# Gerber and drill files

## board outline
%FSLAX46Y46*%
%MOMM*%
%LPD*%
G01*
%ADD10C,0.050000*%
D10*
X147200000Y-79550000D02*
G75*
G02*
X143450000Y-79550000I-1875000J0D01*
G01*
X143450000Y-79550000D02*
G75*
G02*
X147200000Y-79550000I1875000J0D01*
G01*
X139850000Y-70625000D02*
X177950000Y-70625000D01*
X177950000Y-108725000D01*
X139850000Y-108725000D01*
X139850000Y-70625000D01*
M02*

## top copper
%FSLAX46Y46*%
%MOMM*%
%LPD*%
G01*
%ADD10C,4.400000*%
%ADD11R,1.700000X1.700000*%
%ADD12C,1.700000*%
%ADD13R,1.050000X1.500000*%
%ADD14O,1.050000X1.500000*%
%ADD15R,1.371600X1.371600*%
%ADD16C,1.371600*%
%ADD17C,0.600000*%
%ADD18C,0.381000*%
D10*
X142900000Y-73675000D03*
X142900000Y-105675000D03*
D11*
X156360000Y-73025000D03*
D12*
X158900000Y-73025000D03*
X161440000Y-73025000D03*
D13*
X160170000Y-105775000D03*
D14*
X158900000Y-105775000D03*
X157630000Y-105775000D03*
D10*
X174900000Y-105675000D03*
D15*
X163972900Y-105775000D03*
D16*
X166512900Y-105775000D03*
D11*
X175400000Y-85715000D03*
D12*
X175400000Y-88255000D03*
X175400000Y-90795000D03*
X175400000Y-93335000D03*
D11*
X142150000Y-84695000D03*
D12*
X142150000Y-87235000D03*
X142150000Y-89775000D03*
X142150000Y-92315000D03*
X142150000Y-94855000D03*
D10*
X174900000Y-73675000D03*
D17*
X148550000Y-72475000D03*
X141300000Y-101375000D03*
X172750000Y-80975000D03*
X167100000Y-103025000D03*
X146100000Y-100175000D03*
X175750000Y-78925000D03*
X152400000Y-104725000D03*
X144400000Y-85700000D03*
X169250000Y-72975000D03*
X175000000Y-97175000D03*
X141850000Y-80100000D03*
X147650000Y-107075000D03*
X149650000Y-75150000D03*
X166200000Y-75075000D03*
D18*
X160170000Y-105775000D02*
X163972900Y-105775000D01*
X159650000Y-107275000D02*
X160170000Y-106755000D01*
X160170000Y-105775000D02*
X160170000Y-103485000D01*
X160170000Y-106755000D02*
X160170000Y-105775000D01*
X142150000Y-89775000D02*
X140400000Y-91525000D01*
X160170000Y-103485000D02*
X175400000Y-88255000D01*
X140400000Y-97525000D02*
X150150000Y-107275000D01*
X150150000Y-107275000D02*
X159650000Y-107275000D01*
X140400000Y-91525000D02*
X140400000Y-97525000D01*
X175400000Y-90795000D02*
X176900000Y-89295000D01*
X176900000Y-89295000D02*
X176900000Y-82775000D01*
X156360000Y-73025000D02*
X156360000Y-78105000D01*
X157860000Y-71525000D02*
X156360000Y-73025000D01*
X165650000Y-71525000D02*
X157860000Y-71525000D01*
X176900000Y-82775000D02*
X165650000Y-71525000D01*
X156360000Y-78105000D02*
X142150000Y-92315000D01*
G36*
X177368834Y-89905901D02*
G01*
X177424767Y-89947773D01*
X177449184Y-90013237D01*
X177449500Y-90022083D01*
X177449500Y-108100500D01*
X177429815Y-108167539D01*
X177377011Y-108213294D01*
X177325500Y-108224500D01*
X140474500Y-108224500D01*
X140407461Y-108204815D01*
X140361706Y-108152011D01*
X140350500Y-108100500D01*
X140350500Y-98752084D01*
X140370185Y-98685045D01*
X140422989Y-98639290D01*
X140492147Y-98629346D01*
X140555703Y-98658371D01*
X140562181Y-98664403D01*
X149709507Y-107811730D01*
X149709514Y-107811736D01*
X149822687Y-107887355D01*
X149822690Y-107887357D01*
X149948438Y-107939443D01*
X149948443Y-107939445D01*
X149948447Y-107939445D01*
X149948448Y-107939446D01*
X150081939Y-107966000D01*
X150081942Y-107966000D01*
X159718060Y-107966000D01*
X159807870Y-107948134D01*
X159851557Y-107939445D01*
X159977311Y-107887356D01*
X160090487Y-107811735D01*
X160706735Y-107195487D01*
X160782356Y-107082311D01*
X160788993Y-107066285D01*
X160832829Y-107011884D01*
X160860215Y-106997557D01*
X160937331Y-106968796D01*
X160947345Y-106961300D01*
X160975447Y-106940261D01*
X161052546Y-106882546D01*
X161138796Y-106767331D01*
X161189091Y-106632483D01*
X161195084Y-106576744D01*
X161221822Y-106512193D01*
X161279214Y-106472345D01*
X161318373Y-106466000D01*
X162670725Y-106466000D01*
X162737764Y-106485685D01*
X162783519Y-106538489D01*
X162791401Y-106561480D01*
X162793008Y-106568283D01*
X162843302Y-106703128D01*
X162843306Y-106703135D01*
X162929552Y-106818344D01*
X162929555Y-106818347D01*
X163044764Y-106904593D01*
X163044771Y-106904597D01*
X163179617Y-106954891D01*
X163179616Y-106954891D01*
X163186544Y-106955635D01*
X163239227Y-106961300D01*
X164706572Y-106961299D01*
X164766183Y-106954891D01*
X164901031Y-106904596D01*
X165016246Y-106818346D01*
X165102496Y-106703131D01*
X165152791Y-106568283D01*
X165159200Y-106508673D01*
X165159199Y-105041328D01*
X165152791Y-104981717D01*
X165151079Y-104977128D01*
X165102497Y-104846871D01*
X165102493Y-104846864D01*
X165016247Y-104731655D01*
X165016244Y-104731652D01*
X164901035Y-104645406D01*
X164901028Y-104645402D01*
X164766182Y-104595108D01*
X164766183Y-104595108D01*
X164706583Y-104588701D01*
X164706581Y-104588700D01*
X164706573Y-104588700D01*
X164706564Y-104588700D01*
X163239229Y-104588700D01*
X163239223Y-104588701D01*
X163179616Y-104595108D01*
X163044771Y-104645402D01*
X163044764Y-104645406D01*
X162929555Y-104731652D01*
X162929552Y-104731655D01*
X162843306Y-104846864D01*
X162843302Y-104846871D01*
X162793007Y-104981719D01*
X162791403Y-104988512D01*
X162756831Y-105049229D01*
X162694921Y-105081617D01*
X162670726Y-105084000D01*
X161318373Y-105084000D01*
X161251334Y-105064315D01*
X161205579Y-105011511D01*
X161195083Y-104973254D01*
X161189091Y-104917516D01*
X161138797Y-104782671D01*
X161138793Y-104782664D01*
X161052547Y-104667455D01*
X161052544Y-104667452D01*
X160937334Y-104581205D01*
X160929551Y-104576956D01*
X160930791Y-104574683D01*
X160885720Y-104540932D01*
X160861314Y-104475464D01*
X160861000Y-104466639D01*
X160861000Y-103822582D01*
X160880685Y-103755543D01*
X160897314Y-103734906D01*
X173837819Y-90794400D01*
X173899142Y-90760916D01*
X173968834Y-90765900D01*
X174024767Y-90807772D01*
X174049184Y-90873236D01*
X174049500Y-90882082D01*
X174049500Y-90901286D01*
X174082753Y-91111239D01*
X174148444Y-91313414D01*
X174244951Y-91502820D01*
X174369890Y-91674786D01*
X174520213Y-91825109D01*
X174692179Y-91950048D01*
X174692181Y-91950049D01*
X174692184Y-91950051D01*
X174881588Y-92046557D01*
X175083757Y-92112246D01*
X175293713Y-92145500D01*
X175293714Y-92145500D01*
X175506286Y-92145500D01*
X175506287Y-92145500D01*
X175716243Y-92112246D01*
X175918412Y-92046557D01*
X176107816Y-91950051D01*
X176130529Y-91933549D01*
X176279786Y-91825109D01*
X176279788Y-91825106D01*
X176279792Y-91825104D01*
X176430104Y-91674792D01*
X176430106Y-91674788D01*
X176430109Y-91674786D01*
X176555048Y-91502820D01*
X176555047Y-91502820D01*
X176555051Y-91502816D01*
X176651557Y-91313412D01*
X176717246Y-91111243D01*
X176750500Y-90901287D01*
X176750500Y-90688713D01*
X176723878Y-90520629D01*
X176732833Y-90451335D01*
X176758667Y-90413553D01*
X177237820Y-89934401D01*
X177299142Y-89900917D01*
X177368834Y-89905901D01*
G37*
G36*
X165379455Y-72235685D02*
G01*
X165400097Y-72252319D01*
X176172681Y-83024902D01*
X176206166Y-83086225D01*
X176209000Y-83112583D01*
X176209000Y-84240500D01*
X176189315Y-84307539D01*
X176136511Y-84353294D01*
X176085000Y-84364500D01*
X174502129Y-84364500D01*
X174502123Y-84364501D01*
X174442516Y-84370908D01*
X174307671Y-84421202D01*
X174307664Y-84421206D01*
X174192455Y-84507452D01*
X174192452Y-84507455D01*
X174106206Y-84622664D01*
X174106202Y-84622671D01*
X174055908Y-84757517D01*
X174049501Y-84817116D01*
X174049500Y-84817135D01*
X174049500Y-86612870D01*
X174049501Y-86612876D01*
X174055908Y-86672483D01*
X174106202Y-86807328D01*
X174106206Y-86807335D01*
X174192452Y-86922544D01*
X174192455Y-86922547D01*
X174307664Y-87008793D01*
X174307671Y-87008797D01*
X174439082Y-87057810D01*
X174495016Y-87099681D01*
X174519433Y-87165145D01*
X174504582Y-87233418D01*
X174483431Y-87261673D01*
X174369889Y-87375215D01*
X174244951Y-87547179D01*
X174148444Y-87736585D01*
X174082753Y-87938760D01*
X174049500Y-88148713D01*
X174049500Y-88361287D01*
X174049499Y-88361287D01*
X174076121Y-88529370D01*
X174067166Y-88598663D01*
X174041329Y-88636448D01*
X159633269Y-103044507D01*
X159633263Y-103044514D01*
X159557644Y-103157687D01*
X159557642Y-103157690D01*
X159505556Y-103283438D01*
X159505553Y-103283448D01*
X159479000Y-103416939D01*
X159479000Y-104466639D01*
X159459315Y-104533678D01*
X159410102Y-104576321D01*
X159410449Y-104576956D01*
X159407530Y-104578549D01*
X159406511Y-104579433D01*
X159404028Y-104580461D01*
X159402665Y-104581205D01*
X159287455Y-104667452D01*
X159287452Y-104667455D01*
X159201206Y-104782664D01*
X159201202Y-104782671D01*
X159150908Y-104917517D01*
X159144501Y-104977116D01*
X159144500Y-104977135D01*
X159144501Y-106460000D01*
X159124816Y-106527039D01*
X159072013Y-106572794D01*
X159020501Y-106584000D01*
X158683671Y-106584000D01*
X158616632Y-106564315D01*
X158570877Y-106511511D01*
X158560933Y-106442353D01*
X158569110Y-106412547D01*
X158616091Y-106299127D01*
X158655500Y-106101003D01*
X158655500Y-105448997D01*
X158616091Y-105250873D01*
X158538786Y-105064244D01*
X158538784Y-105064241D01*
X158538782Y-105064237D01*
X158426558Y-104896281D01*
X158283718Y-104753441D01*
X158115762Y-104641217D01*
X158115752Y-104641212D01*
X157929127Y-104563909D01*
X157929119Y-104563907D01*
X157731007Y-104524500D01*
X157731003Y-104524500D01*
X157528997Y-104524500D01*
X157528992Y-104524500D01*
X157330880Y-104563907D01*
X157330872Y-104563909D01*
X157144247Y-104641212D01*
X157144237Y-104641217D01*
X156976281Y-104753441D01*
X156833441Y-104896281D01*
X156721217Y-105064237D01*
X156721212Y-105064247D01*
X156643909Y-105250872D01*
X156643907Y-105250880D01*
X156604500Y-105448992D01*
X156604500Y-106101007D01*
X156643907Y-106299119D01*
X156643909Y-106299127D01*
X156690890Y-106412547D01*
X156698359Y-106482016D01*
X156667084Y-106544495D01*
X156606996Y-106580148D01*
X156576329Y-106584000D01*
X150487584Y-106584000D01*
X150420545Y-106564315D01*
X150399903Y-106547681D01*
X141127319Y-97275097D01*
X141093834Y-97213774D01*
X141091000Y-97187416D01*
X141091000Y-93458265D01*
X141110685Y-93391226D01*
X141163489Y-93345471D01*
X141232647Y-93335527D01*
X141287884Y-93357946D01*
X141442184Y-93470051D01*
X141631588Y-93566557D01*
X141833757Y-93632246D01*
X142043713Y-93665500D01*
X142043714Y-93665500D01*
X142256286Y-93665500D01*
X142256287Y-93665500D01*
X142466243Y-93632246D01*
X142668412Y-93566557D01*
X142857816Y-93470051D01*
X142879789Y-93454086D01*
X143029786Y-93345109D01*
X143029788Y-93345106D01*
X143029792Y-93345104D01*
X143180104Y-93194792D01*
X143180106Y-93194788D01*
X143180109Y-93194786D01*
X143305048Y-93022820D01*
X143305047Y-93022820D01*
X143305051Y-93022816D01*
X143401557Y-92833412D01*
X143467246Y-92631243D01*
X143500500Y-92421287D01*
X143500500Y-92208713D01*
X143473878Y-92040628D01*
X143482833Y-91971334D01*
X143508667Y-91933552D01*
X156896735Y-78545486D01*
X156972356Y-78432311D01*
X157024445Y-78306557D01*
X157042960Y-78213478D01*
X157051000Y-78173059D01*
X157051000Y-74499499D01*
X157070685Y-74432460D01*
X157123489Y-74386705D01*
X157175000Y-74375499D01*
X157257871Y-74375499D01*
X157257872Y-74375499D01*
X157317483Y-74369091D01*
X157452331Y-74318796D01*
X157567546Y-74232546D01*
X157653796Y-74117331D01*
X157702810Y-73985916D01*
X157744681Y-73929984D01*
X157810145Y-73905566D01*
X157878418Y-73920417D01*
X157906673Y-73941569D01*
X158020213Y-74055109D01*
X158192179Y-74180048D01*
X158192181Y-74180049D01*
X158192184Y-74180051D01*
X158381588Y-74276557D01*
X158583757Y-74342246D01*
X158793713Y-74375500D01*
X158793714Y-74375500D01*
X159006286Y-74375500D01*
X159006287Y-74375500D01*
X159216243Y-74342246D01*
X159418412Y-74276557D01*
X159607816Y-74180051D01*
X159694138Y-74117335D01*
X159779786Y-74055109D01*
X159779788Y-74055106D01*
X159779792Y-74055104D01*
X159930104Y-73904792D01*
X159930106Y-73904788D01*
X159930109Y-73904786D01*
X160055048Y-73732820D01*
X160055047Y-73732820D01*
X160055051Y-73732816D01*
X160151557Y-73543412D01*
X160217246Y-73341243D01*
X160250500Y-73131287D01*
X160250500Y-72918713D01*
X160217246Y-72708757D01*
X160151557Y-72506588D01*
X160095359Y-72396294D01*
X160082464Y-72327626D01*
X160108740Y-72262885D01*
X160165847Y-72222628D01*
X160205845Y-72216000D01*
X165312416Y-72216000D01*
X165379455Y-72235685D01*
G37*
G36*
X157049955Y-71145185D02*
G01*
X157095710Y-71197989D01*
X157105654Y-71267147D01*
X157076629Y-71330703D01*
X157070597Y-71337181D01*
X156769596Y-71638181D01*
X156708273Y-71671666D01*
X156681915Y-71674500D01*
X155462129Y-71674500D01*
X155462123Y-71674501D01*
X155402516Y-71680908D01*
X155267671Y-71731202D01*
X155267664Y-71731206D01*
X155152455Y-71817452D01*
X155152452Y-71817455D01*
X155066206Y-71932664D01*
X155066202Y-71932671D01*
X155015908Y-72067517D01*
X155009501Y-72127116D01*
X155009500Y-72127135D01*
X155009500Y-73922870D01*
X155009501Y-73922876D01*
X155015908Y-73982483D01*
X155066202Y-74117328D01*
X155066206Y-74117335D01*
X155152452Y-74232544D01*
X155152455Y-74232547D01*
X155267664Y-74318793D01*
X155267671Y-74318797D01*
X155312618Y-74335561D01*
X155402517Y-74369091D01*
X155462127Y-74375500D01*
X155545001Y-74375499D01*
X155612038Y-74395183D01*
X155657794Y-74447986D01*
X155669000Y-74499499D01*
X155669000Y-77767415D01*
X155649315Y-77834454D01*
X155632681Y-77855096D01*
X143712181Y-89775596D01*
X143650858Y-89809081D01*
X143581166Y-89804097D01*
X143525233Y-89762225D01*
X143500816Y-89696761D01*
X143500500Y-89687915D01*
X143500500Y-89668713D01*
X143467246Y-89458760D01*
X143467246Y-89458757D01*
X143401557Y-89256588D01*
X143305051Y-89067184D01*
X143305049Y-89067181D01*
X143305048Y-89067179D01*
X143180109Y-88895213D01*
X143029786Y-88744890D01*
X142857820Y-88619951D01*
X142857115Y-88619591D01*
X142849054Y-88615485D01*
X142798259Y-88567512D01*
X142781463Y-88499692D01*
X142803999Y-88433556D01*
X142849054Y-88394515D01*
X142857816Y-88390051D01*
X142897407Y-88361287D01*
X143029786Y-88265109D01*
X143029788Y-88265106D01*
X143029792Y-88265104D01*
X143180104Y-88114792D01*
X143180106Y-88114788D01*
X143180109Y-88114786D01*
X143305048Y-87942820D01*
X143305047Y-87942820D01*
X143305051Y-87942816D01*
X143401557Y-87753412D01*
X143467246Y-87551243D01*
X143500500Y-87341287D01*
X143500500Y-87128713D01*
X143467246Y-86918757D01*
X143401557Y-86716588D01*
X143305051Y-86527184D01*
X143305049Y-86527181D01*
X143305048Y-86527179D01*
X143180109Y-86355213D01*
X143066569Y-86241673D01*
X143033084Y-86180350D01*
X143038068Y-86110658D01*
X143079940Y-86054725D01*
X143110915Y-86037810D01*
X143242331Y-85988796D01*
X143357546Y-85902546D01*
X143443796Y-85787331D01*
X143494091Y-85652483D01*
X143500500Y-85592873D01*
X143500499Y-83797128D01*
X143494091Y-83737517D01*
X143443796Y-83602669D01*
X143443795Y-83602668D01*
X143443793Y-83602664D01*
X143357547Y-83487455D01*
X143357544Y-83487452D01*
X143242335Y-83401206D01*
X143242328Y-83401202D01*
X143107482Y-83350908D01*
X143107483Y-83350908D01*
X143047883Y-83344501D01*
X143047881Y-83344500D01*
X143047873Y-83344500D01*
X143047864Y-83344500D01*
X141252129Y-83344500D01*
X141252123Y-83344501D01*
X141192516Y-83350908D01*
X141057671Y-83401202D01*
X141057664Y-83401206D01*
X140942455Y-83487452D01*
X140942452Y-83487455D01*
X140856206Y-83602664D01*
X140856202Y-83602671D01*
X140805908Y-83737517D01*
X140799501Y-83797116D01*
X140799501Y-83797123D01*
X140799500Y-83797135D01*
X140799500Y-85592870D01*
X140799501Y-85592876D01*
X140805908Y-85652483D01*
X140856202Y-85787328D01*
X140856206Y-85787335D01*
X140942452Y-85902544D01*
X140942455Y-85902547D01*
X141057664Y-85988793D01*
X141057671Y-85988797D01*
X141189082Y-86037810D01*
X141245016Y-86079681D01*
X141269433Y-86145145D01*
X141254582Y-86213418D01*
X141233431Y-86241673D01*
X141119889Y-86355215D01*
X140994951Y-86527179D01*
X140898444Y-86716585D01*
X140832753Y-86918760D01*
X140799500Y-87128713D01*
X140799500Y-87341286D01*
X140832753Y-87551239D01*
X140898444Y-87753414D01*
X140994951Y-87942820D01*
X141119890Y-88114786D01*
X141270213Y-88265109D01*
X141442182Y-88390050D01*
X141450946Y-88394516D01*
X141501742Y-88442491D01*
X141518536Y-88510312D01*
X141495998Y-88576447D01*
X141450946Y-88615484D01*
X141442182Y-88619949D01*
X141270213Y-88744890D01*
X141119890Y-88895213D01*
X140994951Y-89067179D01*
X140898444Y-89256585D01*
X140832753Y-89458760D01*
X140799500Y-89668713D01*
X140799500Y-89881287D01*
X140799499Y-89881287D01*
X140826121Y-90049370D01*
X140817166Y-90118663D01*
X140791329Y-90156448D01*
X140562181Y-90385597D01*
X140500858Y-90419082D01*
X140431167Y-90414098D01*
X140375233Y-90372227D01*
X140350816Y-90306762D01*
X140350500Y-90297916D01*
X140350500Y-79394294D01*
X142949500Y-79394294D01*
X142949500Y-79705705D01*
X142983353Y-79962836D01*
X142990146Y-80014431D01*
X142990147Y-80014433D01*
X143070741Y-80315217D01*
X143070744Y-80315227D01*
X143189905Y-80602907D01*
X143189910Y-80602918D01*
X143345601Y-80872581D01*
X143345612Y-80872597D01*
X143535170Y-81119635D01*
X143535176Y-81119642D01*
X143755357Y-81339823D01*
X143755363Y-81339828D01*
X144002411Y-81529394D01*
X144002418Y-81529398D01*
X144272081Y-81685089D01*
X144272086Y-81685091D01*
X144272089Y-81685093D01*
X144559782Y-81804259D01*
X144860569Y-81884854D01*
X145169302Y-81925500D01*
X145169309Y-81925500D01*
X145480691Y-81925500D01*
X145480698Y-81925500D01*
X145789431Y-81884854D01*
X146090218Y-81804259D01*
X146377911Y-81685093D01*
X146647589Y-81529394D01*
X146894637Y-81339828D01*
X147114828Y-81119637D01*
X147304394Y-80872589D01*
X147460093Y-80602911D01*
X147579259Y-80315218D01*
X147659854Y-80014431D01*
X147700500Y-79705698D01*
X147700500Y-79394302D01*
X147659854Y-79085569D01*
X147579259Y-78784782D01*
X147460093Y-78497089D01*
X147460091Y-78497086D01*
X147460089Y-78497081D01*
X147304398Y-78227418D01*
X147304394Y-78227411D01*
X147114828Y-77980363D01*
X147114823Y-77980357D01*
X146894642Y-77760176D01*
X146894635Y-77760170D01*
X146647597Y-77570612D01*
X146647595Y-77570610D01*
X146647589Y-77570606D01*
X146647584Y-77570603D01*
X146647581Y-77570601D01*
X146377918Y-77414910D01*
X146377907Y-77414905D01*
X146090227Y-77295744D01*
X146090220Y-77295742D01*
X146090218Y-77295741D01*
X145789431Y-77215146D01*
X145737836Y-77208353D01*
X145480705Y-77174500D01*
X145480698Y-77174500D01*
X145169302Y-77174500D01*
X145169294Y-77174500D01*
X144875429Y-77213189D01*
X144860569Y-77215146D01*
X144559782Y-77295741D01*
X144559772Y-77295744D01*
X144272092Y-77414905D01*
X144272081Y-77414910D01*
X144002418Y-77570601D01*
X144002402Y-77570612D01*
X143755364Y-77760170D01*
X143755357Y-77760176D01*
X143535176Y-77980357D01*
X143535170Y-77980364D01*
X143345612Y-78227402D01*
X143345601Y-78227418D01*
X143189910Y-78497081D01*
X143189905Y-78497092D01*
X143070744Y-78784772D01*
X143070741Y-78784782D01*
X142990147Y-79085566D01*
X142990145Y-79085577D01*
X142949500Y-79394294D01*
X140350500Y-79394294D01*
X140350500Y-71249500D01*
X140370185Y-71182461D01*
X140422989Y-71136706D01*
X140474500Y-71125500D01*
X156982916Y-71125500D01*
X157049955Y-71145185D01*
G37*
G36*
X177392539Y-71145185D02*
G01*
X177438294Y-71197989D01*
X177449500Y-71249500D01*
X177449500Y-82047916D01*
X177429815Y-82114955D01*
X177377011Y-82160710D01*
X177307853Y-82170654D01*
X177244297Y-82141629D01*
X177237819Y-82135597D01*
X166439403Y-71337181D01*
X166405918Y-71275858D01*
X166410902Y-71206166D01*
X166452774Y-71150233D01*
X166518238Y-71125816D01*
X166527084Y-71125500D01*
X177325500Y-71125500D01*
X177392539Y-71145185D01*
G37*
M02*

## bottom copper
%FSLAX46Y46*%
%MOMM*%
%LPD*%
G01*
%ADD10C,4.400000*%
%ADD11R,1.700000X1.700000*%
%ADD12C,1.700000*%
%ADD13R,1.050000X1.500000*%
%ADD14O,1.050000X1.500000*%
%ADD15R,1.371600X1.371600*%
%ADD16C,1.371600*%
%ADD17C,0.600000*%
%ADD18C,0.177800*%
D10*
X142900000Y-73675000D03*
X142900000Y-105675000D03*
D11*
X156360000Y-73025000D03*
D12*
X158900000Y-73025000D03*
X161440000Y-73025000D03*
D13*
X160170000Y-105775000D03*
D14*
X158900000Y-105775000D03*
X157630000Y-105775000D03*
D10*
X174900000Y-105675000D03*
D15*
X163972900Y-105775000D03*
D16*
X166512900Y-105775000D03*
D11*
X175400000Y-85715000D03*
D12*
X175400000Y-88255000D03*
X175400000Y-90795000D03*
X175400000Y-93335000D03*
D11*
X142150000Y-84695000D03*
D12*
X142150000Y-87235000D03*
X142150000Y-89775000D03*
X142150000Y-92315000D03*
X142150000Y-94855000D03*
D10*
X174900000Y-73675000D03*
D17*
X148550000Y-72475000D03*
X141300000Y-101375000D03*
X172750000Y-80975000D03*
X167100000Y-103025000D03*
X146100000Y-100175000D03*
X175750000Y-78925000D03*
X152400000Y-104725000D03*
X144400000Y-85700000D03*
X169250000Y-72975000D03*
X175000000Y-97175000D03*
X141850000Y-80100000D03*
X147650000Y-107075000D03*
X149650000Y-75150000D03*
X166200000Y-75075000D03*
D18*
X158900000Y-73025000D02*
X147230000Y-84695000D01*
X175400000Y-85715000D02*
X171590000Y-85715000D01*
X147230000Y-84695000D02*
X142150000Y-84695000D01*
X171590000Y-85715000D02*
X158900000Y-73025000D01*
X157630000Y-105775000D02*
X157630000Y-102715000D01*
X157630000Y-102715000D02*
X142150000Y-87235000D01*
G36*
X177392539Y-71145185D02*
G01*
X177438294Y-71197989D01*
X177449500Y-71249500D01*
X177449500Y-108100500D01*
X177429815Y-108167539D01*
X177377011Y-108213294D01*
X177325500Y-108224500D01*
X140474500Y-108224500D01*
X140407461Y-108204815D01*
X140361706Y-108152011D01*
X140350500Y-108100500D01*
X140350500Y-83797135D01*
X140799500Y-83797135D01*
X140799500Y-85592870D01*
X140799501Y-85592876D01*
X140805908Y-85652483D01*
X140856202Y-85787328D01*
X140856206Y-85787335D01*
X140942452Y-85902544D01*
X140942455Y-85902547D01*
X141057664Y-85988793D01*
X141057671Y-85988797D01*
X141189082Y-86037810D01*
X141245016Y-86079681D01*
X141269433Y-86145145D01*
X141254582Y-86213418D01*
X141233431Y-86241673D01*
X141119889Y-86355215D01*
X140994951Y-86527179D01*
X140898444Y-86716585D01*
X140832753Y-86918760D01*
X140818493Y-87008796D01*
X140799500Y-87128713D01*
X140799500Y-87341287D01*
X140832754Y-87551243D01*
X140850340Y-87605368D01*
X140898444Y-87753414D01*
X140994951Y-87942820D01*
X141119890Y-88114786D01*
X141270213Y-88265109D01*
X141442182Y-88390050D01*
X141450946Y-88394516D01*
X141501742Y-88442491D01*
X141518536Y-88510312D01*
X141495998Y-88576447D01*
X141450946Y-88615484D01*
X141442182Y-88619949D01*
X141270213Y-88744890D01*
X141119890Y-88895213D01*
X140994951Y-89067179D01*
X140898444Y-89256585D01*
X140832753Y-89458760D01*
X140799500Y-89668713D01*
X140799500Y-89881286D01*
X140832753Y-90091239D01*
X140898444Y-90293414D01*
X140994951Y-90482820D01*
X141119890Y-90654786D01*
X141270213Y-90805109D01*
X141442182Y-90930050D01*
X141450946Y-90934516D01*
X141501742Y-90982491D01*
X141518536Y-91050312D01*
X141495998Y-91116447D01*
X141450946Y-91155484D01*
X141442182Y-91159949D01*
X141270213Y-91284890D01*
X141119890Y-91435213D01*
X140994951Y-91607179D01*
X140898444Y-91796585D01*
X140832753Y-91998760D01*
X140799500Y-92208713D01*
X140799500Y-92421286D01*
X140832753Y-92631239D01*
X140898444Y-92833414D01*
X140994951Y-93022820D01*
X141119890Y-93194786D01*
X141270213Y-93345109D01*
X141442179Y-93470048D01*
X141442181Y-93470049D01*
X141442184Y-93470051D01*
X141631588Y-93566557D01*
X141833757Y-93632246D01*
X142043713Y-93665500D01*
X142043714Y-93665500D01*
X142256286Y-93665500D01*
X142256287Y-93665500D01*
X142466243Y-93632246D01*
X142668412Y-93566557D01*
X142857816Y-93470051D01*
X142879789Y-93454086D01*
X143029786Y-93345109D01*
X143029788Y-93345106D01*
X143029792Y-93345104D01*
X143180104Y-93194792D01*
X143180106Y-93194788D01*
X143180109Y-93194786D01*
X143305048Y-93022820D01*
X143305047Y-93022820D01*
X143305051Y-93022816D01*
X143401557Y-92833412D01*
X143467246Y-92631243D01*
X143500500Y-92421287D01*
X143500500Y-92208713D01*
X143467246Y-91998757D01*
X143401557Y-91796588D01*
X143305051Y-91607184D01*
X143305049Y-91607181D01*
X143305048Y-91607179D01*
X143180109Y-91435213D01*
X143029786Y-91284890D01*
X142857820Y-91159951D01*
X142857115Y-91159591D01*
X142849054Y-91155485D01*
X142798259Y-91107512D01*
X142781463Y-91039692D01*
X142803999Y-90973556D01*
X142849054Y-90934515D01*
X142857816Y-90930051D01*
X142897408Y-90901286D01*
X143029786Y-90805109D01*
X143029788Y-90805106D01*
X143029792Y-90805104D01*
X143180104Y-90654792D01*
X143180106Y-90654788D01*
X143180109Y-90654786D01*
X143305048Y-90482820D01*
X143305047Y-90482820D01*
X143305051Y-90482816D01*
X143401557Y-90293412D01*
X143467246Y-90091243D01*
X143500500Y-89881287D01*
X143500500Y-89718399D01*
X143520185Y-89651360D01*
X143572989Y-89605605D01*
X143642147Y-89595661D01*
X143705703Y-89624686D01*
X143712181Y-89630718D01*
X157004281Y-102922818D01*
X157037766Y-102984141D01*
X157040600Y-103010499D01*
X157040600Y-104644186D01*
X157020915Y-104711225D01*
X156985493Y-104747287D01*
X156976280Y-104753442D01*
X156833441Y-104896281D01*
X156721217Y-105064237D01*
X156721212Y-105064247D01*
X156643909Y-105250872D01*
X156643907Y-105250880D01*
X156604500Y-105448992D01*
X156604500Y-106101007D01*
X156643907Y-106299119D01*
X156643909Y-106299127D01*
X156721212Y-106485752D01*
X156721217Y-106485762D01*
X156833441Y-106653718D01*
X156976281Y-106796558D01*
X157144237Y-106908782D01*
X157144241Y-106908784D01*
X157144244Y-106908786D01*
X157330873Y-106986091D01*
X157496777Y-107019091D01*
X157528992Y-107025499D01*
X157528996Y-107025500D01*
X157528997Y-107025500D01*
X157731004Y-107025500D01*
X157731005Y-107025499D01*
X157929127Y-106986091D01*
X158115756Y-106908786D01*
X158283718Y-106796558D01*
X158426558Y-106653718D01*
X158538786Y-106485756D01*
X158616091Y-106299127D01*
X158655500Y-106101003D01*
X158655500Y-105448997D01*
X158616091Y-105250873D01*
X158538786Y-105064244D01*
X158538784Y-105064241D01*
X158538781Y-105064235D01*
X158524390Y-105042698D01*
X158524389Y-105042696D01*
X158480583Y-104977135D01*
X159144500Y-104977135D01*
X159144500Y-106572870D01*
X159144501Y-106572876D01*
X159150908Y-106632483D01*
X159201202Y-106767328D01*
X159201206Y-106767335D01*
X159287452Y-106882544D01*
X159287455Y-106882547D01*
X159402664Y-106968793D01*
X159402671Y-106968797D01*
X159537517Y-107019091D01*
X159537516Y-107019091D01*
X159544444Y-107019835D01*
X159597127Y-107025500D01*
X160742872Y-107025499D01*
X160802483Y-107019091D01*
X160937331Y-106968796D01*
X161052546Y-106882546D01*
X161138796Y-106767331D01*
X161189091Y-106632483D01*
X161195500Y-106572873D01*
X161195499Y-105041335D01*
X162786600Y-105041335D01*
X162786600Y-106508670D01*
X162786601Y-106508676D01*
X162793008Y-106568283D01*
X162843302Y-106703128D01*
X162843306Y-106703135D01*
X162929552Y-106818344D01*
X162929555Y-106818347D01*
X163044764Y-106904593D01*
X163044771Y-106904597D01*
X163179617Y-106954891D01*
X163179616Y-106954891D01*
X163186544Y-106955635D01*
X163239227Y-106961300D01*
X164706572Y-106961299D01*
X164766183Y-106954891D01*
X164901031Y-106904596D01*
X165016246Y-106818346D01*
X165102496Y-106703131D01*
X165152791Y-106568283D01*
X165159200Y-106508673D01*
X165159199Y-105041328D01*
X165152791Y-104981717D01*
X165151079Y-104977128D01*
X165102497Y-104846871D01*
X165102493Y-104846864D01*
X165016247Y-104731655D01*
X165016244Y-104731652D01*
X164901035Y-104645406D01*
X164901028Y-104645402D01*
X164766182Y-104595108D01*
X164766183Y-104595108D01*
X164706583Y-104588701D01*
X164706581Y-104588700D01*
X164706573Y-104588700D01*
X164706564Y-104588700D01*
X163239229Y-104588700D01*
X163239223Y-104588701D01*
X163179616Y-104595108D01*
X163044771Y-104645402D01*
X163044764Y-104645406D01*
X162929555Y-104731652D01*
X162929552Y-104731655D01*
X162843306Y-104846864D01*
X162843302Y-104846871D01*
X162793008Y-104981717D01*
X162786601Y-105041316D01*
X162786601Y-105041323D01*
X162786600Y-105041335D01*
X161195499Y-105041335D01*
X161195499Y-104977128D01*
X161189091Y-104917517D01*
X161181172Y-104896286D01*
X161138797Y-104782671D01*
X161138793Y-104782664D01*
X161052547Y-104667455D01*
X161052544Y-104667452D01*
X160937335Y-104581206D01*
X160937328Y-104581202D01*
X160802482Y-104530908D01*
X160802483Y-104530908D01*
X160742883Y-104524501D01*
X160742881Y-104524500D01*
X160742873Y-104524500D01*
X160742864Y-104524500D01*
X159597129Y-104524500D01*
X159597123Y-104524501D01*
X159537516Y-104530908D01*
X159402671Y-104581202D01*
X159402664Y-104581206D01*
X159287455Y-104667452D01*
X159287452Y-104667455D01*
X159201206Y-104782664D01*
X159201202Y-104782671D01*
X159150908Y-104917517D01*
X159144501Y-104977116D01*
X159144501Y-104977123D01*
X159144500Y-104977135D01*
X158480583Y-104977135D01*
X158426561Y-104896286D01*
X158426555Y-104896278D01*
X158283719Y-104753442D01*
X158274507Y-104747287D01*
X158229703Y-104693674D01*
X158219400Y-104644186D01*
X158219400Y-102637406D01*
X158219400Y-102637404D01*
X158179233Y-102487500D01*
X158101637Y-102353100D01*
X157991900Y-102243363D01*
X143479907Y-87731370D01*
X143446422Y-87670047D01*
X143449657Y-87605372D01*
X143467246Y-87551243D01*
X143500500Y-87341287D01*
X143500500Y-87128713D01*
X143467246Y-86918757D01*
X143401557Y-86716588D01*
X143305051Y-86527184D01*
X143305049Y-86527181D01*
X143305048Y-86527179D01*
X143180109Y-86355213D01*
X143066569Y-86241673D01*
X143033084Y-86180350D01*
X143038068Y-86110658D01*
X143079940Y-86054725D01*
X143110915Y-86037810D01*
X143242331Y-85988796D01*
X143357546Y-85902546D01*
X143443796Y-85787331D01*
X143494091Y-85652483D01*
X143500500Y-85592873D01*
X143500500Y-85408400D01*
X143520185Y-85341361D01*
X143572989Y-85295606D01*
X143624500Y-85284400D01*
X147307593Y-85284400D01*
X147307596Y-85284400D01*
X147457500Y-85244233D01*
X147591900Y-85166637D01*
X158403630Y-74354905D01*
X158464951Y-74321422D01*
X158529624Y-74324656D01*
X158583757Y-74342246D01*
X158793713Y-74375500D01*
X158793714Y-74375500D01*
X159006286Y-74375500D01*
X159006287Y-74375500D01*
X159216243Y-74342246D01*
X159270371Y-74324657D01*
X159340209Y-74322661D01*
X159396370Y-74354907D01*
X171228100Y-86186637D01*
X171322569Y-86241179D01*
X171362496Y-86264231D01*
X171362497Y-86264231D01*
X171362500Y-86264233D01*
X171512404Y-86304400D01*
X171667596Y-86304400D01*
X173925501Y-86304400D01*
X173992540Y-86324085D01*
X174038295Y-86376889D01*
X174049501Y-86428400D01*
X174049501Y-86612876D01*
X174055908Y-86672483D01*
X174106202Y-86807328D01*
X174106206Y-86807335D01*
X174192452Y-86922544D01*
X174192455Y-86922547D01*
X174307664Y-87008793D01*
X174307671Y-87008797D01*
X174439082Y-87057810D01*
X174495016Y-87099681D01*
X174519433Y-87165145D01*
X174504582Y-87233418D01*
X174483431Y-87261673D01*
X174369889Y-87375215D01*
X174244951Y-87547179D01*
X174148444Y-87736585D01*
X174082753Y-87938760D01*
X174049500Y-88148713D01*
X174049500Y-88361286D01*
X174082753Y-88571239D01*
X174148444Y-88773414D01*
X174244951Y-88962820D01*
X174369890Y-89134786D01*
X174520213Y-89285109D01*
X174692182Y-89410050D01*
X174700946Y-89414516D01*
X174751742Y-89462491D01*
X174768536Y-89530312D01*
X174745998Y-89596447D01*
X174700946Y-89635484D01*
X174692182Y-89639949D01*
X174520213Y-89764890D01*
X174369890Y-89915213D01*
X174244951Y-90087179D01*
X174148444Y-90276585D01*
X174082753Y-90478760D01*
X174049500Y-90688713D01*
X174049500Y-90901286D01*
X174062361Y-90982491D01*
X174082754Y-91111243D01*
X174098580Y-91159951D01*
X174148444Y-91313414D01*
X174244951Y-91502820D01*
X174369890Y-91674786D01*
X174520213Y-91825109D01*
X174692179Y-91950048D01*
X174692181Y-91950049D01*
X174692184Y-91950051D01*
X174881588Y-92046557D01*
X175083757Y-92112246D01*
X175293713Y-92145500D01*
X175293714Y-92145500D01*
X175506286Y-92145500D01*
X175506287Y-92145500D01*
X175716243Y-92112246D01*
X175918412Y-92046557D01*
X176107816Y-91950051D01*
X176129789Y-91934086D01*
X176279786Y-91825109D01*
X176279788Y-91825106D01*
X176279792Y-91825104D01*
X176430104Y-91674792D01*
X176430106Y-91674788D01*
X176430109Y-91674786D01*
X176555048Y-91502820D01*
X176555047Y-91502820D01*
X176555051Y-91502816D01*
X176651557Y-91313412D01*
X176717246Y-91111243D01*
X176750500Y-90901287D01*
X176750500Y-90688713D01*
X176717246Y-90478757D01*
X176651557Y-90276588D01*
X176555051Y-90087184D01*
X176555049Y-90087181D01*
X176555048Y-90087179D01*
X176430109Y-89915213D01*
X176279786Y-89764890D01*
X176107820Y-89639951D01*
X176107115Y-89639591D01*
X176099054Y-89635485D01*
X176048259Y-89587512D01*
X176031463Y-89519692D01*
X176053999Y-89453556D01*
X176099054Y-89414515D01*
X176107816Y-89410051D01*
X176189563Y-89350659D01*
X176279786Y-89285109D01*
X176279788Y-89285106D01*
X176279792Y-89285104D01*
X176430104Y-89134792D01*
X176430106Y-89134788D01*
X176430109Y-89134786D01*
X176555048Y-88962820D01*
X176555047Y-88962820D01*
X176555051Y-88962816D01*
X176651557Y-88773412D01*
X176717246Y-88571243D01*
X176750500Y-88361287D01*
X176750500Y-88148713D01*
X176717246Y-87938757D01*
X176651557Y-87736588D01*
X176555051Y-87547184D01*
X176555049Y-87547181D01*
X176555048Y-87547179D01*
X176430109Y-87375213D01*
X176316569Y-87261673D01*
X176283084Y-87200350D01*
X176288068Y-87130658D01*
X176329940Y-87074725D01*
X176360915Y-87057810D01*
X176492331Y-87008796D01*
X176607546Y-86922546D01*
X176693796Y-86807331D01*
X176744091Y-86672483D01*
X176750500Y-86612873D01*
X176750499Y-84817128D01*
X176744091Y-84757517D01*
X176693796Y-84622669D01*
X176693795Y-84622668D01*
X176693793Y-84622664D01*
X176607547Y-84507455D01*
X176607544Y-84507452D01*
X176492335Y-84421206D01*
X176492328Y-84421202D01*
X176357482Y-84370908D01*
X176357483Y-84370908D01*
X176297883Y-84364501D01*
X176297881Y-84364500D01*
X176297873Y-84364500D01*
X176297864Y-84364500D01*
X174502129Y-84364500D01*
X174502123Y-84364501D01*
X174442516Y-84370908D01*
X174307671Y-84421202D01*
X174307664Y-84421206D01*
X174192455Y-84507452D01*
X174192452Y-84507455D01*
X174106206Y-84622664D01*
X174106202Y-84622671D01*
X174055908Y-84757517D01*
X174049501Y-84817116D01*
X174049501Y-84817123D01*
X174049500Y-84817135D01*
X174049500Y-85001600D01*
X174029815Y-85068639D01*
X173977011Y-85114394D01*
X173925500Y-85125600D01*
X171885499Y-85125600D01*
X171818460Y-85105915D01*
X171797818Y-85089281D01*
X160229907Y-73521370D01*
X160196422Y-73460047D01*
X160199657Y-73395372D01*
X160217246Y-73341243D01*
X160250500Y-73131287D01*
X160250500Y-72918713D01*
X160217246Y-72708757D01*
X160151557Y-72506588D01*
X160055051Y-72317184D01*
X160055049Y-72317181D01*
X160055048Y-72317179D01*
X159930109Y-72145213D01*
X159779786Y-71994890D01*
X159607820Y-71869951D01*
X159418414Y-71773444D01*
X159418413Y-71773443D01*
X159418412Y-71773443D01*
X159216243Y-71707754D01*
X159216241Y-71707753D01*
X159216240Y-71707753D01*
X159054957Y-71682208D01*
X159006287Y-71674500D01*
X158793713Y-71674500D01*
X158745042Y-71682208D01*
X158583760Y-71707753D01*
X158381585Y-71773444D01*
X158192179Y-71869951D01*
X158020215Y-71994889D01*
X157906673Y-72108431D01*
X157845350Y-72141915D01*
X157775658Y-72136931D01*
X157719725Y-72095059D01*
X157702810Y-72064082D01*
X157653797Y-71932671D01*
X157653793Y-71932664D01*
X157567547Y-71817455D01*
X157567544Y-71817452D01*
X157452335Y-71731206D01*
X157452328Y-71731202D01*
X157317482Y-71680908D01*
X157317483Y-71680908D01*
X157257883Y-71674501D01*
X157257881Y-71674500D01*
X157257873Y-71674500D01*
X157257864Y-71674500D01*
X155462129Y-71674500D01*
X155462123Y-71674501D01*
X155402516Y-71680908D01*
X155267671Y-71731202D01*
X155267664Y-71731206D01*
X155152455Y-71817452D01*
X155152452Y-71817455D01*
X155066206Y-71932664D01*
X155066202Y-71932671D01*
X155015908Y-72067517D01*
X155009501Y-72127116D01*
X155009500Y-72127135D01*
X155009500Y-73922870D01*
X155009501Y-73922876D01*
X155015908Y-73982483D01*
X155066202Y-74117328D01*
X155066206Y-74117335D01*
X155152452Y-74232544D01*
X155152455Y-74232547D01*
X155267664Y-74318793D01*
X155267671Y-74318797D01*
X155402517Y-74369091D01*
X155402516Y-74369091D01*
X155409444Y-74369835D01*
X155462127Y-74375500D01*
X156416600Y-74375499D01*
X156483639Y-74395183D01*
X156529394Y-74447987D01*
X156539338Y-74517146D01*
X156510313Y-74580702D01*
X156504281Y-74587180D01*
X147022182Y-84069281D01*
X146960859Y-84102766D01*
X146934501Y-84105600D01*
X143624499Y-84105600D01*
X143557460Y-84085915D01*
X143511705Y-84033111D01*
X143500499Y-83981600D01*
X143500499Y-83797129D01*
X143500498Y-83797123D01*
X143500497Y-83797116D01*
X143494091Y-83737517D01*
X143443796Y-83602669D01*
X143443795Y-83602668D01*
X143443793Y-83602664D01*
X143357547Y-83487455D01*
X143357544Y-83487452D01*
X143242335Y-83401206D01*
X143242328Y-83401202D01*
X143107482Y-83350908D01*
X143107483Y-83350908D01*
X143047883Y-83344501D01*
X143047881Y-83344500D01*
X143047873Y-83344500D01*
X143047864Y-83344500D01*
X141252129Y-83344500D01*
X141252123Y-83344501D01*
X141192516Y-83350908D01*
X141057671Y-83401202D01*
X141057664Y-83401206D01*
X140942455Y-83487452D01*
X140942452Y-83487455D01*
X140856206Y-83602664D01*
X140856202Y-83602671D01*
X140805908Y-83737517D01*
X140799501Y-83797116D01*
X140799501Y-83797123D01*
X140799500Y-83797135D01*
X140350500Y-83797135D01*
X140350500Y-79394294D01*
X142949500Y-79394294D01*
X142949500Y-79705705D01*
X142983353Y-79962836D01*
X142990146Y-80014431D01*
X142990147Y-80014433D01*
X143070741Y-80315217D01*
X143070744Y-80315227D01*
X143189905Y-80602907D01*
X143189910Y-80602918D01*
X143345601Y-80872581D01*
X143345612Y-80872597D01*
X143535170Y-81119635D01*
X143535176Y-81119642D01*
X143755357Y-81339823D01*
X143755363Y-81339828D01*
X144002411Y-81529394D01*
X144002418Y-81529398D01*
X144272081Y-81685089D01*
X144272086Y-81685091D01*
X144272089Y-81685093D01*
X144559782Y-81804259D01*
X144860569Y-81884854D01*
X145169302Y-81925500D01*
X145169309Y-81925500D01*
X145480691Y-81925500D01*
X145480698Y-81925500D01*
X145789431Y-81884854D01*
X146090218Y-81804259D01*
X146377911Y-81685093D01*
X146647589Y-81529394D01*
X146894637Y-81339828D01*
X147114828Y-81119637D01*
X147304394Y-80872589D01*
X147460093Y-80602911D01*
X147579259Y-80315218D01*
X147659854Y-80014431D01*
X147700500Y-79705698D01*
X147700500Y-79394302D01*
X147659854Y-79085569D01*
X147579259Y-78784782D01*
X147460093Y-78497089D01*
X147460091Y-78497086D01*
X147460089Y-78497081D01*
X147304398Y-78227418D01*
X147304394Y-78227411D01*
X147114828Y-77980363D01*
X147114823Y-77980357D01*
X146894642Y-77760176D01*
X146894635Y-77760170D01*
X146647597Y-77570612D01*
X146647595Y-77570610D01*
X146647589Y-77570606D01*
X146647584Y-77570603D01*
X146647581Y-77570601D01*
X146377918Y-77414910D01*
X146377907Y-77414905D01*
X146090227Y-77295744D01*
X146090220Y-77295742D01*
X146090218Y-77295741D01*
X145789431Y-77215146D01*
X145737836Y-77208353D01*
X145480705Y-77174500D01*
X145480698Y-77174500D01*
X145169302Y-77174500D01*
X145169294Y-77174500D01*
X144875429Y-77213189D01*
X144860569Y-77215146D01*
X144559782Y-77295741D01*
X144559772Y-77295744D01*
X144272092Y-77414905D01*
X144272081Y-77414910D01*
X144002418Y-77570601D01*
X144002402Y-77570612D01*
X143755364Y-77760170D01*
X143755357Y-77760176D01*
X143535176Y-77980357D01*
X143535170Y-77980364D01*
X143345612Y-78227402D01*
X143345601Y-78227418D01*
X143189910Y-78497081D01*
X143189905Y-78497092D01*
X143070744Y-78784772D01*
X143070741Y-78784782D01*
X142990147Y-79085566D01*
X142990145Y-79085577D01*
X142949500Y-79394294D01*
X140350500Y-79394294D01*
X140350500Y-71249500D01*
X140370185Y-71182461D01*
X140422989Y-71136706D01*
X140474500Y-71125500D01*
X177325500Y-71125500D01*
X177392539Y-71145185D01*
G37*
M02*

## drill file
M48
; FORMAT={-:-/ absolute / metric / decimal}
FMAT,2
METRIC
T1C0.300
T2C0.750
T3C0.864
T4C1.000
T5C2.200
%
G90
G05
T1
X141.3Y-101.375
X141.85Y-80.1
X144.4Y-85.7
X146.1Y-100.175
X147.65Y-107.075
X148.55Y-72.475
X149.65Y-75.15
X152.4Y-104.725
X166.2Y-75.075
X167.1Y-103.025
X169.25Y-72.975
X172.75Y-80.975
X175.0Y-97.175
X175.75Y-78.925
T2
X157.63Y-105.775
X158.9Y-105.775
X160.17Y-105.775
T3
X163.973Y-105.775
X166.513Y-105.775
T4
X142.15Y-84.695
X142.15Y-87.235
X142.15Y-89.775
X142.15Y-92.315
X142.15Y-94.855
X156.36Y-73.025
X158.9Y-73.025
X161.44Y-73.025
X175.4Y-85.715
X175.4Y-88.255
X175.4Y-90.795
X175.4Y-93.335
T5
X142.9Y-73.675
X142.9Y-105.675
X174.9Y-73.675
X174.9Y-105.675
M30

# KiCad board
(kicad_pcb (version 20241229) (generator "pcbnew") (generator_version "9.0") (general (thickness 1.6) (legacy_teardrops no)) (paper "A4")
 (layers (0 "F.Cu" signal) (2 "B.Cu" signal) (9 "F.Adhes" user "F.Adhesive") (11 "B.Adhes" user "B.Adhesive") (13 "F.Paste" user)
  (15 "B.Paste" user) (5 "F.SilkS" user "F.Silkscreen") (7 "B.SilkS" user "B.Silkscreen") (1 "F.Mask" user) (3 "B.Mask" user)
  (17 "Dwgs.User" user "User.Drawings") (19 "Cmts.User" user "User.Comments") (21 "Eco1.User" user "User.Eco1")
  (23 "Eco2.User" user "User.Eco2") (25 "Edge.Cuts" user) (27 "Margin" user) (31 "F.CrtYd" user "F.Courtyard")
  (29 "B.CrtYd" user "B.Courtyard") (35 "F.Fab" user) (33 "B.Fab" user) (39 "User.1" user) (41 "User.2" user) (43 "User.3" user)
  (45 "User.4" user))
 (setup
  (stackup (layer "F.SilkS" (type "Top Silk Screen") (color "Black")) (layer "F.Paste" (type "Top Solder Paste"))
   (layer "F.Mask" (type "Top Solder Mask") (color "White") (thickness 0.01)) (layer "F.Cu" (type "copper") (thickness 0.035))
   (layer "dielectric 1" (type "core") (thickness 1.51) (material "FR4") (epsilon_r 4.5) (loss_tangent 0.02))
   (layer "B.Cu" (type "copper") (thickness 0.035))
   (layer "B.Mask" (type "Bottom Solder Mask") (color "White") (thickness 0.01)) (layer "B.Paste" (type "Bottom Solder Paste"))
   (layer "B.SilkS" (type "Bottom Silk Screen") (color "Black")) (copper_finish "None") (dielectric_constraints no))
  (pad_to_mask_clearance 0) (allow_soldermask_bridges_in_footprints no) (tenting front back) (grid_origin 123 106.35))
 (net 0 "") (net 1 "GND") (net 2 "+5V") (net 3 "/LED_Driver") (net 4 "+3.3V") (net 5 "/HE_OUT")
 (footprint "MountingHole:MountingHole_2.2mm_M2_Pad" (layer "F.Cu") (at 142.9 73.675)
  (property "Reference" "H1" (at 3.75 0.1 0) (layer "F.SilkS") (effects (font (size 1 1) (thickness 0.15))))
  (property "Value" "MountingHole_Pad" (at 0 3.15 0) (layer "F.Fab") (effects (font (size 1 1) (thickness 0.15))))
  (pad "1" thru_hole circle (at 0 0) (size 4.4 4.4) (drill 2.2) (layers "*.Cu" "*.Mask") (remove_unused_layers no) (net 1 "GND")
   (zone_connect 2)))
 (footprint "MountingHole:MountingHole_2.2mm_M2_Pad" (layer "F.Cu") (at 142.9 105.675)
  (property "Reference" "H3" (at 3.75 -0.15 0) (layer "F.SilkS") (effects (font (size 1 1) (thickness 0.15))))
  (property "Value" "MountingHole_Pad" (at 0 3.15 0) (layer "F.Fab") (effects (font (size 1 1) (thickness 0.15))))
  (pad "1" thru_hole circle (at 0 0) (size 4.4 4.4) (drill 2.2) (layers "*.Cu" "*.Mask") (remove_unused_layers no) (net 1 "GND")
   (zone_connect 2)))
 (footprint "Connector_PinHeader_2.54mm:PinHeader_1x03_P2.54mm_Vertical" (layer "F.Cu") (at 156.36 73.025 90)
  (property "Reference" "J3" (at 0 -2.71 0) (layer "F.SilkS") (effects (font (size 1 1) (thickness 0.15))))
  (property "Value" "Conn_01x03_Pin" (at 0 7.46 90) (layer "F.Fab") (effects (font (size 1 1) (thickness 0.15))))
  (pad "1" thru_hole rect (at 0 0 90) (size 1.7 1.7) (drill 1) (layers "*.Cu" "*.Mask") (remove_unused_layers no) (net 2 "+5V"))
  (pad "2" thru_hole circle (at 0 2.54 90) (size 1.7 1.7) (drill 1) (layers "*.Cu" "*.Mask") (remove_unused_layers no) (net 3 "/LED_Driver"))
  (pad "3" thru_hole circle (at 0 5.08 90) (size 1.7 1.7) (drill 1) (layers "*.Cu" "*.Mask") (remove_unused_layers no) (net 1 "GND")))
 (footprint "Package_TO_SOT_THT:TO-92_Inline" (layer "F.Cu") (at 160.17 105.775 180)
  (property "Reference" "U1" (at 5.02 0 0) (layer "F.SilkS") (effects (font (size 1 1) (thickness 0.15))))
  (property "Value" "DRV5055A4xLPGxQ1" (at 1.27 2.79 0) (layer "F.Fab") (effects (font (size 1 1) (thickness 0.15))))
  (pad "1" thru_hole rect (at 0 0 180) (size 1.05 1.5) (drill 0.75) (layers "*.Cu" "*.Mask") (remove_unused_layers no) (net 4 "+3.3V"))
  (pad "2" thru_hole oval (at 1.27 0 180) (size 1.05 1.5) (drill 0.75) (layers "*.Cu" "*.Mask") (remove_unused_layers no) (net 1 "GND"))
  (pad "3" thru_hole oval (at 2.54 0 180) (size 1.05 1.5) (drill 0.75) (layers "*.Cu" "*.Mask") (remove_unused_layers no) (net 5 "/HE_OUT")))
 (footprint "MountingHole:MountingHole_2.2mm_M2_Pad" (layer "F.Cu") (at 174.9 105.675)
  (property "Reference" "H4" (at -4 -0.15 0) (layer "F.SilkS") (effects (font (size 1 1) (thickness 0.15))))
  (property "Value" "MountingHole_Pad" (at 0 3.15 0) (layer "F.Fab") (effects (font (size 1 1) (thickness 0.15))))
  (pad "1" thru_hole circle (at 0 0) (size 4.4 4.4) (drill 2.2) (layers "*.Cu" "*.Mask") (remove_unused_layers no) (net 1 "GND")
   (zone_connect 2)))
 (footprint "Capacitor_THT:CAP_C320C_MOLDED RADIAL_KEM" (layer "F.Cu") (at 163.9729 105.775)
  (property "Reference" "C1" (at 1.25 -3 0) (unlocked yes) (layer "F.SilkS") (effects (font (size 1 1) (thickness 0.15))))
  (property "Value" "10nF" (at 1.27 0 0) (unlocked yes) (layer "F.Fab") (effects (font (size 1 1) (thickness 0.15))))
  (pad "1" thru_hole rect (at 0 0) (size 1.3716 1.3716) (drill 0.8636) (layers "*.Cu" "*.Mask") (remove_unused_layers no) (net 4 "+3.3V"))
  (pad "2" thru_hole circle (at 2.54 0) (size 1.3716 1.3716) (drill 0.8636) (layers "*.Cu" "*.Mask") (remove_unused_layers no) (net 1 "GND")))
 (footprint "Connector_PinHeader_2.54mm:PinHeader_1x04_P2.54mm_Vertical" (layer "F.Cu") (at 175.4 85.715)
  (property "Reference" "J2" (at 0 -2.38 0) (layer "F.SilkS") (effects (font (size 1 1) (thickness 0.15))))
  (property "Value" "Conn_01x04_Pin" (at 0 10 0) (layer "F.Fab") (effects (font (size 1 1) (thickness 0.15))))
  (pad "1" thru_hole rect (at 0 0) (size 1.7 1.7) (drill 1) (layers "*.Cu" "*.Mask") (remove_unused_layers no) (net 3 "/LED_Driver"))
  (pad "2" thru_hole circle (at 0 2.54) (size 1.7 1.7) (drill 1) (layers "*.Cu" "*.Mask") (remove_unused_layers no) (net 4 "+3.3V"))
  (pad "3" thru_hole circle (at 0 5.08) (size 1.7 1.7) (drill 1) (layers "*.Cu" "*.Mask") (remove_unused_layers no) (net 2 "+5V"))
  (pad "4" thru_hole circle (at 0 7.62) (size 1.7 1.7) (drill 1) (layers "*.Cu" "*.Mask") (remove_unused_layers no) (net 1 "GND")))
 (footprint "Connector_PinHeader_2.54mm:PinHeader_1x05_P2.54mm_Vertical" (layer "F.Cu") (at 142.15 84.695)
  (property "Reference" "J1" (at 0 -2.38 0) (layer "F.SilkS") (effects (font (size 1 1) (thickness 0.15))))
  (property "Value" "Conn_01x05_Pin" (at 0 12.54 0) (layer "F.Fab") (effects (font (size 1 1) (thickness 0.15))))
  (pad "1" thru_hole rect (at 0 0) (size 1.7 1.7) (drill 1) (layers "*.Cu" "*.Mask") (remove_unused_layers no) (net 3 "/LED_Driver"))
  (pad "2" thru_hole circle (at 0 2.54) (size 1.7 1.7) (drill 1) (layers "*.Cu" "*.Mask") (remove_unused_layers no) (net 5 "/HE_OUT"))
  (pad "3" thru_hole circle (at 0 5.08) (size 1.7 1.7) (drill 1) (layers "*.Cu" "*.Mask") (remove_unused_layers no) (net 4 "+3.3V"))
  (pad "4" thru_hole circle (at 0 7.62) (size 1.7 1.7) (drill 1) (layers "*.Cu" "*.Mask") (remove_unused_layers no) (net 2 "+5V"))
  (pad "5" thru_hole circle (at 0 10.16) (size 1.7 1.7) (drill 1) (layers "*.Cu" "*.Mask") (remove_unused_layers no) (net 1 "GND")))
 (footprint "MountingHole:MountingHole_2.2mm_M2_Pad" (layer "F.Cu") (at 174.9 73.675)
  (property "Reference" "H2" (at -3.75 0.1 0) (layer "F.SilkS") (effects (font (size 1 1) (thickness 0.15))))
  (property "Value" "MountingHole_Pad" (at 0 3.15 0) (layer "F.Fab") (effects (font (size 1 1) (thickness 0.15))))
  (pad "1" thru_hole circle (at 0 0) (size 4.4 4.4) (drill 2.2) (layers "*.Cu" "*.Mask") (remove_unused_layers no) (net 1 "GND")
   (zone_connect 2)))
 (gr_circle (center 145.325 79.55) (end 147.2 79.55) (stroke (width 0.05) (type solid)) (fill no) (layer "Edge.Cuts"))
 (gr_rect (start 139.85 70.625) (end 177.95 108.725) (stroke (width 0.05) (type solid)) (fill no) (locked yes) (layer "Edge.Cuts"))
 (segment (start 160.17 105.775) (end 163.9729 105.775) (width 0.381) (layer "F.Cu") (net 4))
 (segment (start 159.65 107.275) (end 160.17 106.755) (width 0.381) (layer "F.Cu") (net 4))
 (segment (start 160.17 105.775) (end 160.17 103.485) (width 0.381) (layer "F.Cu") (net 4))
 (segment (start 160.17 106.755) (end 160.17 105.775) (width 0.381) (layer "F.Cu") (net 4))
 (segment (start 142.15 89.775) (end 140.4 91.525) (width 0.381) (layer "F.Cu") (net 4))
 (segment (start 160.17 103.485) (end 175.4 88.255) (width 0.381) (layer "F.Cu") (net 4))
 (segment (start 140.4 97.525) (end 150.15 107.275) (width 0.381) (layer "F.Cu") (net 4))
 (segment (start 150.15 107.275) (end 159.65 107.275) (width 0.381) (layer "F.Cu") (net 4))
 (segment (start 140.4 91.525) (end 140.4 97.525) (width 0.381) (layer "F.Cu") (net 4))
 (via (at 148.55 72.475) (size 0.6) (drill 0.3) (layers "F.Cu" "B.Cu") (free yes) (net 1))
 (via (at 141.3 101.375) (size 0.6) (drill 0.3) (layers "F.Cu" "B.Cu") (free yes) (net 1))
 (via (at 172.75 80.975) (size 0.6) (drill 0.3) (layers "F.Cu" "B.Cu") (free yes) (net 1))
 (via (at 167.1 103.025) (size 0.6) (drill 0.3) (layers "F.Cu" "B.Cu") (free yes) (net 1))
 (via (at 146.1 100.175) (size 0.6) (drill 0.3) (layers "F.Cu" "B.Cu") (free yes) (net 1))
 (via (at 175.75 78.925) (size 0.6) (drill 0.3) (layers "F.Cu" "B.Cu") (free yes) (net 1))
 (via (at 152.4 104.725) (size 0.6) (drill 0.3) (layers "F.Cu" "B.Cu") (free yes) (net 1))
 (via (at 144.4 85.7) (size 0.6) (drill 0.3) (layers "F.Cu" "B.Cu") (free yes) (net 1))
 (via (at 169.25 72.975) (size 0.6) (drill 0.3) (layers "F.Cu" "B.Cu") (free yes) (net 1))
 (via (at 175 97.175) (size 0.6) (drill 0.3) (layers "F.Cu" "B.Cu") (free yes) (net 1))
 (via (at 141.85 80.1) (size 0.6) (drill 0.3) (layers "F.Cu" "B.Cu") (free yes) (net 1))
 (via (at 147.65 107.075) (size 0.6) (drill 0.3) (layers "F.Cu" "B.Cu") (free yes) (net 1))
 (via (at 149.65 75.15) (size 0.6) (drill 0.3) (layers "F.Cu" "B.Cu") (free yes) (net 1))
 (via (at 166.2 75.075) (size 0.6) (drill 0.3) (layers "F.Cu" "B.Cu") (free yes) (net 1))
 (segment (start 158.9 73.025) (end 147.23 84.695) (width 0.1778) (layer "B.Cu") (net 3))
 (segment (start 175.4 85.715) (end 171.59 85.715) (width 0.1778) (layer "B.Cu") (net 3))
 (segment (start 147.23 84.695) (end 142.15 84.695) (width 0.1778) (layer "B.Cu") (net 3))
 (segment (start 171.59 85.715) (end 158.9 73.025) (width 0.1778) (layer "B.Cu") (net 3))
 (segment (start 175.4 90.795) (end 176.9 89.295) (width 0.381) (layer "F.Cu") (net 2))
 (segment (start 176.9 89.295) (end 176.9 82.775) (width 0.381) (layer "F.Cu") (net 2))
 (segment (start 156.36 73.025) (end 156.36 78.105) (width 0.381) (layer "F.Cu") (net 2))
 (segment (start 157.86 71.525) (end 156.36 73.025) (width 0.381) (layer "F.Cu") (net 2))
 (segment (start 165.65 71.525) (end 157.86 71.525) (width 0.381) (layer "F.Cu") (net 2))
 (segment (start 176.9 82.775) (end 165.65 71.525) (width 0.381) (layer "F.Cu") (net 2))
 (segment (start 156.36 78.105) (end 142.15 92.315) (width 0.381) (layer "F.Cu") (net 2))
 (segment (start 157.63 105.775) (end 157.63 102.715) (width 0.1778) (layer "B.Cu") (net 5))
 (segment (start 157.63 102.715) (end 142.15 87.235) (width 0.1778) (layer "B.Cu") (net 5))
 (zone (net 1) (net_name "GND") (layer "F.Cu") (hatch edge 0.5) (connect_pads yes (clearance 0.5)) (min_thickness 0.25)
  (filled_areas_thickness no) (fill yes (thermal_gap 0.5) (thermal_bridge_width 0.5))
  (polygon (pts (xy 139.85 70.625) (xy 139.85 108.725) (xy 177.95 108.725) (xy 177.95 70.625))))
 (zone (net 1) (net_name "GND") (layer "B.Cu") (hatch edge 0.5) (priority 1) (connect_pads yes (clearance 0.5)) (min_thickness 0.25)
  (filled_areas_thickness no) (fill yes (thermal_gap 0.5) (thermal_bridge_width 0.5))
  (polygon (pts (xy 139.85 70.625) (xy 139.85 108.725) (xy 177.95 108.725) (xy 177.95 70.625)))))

